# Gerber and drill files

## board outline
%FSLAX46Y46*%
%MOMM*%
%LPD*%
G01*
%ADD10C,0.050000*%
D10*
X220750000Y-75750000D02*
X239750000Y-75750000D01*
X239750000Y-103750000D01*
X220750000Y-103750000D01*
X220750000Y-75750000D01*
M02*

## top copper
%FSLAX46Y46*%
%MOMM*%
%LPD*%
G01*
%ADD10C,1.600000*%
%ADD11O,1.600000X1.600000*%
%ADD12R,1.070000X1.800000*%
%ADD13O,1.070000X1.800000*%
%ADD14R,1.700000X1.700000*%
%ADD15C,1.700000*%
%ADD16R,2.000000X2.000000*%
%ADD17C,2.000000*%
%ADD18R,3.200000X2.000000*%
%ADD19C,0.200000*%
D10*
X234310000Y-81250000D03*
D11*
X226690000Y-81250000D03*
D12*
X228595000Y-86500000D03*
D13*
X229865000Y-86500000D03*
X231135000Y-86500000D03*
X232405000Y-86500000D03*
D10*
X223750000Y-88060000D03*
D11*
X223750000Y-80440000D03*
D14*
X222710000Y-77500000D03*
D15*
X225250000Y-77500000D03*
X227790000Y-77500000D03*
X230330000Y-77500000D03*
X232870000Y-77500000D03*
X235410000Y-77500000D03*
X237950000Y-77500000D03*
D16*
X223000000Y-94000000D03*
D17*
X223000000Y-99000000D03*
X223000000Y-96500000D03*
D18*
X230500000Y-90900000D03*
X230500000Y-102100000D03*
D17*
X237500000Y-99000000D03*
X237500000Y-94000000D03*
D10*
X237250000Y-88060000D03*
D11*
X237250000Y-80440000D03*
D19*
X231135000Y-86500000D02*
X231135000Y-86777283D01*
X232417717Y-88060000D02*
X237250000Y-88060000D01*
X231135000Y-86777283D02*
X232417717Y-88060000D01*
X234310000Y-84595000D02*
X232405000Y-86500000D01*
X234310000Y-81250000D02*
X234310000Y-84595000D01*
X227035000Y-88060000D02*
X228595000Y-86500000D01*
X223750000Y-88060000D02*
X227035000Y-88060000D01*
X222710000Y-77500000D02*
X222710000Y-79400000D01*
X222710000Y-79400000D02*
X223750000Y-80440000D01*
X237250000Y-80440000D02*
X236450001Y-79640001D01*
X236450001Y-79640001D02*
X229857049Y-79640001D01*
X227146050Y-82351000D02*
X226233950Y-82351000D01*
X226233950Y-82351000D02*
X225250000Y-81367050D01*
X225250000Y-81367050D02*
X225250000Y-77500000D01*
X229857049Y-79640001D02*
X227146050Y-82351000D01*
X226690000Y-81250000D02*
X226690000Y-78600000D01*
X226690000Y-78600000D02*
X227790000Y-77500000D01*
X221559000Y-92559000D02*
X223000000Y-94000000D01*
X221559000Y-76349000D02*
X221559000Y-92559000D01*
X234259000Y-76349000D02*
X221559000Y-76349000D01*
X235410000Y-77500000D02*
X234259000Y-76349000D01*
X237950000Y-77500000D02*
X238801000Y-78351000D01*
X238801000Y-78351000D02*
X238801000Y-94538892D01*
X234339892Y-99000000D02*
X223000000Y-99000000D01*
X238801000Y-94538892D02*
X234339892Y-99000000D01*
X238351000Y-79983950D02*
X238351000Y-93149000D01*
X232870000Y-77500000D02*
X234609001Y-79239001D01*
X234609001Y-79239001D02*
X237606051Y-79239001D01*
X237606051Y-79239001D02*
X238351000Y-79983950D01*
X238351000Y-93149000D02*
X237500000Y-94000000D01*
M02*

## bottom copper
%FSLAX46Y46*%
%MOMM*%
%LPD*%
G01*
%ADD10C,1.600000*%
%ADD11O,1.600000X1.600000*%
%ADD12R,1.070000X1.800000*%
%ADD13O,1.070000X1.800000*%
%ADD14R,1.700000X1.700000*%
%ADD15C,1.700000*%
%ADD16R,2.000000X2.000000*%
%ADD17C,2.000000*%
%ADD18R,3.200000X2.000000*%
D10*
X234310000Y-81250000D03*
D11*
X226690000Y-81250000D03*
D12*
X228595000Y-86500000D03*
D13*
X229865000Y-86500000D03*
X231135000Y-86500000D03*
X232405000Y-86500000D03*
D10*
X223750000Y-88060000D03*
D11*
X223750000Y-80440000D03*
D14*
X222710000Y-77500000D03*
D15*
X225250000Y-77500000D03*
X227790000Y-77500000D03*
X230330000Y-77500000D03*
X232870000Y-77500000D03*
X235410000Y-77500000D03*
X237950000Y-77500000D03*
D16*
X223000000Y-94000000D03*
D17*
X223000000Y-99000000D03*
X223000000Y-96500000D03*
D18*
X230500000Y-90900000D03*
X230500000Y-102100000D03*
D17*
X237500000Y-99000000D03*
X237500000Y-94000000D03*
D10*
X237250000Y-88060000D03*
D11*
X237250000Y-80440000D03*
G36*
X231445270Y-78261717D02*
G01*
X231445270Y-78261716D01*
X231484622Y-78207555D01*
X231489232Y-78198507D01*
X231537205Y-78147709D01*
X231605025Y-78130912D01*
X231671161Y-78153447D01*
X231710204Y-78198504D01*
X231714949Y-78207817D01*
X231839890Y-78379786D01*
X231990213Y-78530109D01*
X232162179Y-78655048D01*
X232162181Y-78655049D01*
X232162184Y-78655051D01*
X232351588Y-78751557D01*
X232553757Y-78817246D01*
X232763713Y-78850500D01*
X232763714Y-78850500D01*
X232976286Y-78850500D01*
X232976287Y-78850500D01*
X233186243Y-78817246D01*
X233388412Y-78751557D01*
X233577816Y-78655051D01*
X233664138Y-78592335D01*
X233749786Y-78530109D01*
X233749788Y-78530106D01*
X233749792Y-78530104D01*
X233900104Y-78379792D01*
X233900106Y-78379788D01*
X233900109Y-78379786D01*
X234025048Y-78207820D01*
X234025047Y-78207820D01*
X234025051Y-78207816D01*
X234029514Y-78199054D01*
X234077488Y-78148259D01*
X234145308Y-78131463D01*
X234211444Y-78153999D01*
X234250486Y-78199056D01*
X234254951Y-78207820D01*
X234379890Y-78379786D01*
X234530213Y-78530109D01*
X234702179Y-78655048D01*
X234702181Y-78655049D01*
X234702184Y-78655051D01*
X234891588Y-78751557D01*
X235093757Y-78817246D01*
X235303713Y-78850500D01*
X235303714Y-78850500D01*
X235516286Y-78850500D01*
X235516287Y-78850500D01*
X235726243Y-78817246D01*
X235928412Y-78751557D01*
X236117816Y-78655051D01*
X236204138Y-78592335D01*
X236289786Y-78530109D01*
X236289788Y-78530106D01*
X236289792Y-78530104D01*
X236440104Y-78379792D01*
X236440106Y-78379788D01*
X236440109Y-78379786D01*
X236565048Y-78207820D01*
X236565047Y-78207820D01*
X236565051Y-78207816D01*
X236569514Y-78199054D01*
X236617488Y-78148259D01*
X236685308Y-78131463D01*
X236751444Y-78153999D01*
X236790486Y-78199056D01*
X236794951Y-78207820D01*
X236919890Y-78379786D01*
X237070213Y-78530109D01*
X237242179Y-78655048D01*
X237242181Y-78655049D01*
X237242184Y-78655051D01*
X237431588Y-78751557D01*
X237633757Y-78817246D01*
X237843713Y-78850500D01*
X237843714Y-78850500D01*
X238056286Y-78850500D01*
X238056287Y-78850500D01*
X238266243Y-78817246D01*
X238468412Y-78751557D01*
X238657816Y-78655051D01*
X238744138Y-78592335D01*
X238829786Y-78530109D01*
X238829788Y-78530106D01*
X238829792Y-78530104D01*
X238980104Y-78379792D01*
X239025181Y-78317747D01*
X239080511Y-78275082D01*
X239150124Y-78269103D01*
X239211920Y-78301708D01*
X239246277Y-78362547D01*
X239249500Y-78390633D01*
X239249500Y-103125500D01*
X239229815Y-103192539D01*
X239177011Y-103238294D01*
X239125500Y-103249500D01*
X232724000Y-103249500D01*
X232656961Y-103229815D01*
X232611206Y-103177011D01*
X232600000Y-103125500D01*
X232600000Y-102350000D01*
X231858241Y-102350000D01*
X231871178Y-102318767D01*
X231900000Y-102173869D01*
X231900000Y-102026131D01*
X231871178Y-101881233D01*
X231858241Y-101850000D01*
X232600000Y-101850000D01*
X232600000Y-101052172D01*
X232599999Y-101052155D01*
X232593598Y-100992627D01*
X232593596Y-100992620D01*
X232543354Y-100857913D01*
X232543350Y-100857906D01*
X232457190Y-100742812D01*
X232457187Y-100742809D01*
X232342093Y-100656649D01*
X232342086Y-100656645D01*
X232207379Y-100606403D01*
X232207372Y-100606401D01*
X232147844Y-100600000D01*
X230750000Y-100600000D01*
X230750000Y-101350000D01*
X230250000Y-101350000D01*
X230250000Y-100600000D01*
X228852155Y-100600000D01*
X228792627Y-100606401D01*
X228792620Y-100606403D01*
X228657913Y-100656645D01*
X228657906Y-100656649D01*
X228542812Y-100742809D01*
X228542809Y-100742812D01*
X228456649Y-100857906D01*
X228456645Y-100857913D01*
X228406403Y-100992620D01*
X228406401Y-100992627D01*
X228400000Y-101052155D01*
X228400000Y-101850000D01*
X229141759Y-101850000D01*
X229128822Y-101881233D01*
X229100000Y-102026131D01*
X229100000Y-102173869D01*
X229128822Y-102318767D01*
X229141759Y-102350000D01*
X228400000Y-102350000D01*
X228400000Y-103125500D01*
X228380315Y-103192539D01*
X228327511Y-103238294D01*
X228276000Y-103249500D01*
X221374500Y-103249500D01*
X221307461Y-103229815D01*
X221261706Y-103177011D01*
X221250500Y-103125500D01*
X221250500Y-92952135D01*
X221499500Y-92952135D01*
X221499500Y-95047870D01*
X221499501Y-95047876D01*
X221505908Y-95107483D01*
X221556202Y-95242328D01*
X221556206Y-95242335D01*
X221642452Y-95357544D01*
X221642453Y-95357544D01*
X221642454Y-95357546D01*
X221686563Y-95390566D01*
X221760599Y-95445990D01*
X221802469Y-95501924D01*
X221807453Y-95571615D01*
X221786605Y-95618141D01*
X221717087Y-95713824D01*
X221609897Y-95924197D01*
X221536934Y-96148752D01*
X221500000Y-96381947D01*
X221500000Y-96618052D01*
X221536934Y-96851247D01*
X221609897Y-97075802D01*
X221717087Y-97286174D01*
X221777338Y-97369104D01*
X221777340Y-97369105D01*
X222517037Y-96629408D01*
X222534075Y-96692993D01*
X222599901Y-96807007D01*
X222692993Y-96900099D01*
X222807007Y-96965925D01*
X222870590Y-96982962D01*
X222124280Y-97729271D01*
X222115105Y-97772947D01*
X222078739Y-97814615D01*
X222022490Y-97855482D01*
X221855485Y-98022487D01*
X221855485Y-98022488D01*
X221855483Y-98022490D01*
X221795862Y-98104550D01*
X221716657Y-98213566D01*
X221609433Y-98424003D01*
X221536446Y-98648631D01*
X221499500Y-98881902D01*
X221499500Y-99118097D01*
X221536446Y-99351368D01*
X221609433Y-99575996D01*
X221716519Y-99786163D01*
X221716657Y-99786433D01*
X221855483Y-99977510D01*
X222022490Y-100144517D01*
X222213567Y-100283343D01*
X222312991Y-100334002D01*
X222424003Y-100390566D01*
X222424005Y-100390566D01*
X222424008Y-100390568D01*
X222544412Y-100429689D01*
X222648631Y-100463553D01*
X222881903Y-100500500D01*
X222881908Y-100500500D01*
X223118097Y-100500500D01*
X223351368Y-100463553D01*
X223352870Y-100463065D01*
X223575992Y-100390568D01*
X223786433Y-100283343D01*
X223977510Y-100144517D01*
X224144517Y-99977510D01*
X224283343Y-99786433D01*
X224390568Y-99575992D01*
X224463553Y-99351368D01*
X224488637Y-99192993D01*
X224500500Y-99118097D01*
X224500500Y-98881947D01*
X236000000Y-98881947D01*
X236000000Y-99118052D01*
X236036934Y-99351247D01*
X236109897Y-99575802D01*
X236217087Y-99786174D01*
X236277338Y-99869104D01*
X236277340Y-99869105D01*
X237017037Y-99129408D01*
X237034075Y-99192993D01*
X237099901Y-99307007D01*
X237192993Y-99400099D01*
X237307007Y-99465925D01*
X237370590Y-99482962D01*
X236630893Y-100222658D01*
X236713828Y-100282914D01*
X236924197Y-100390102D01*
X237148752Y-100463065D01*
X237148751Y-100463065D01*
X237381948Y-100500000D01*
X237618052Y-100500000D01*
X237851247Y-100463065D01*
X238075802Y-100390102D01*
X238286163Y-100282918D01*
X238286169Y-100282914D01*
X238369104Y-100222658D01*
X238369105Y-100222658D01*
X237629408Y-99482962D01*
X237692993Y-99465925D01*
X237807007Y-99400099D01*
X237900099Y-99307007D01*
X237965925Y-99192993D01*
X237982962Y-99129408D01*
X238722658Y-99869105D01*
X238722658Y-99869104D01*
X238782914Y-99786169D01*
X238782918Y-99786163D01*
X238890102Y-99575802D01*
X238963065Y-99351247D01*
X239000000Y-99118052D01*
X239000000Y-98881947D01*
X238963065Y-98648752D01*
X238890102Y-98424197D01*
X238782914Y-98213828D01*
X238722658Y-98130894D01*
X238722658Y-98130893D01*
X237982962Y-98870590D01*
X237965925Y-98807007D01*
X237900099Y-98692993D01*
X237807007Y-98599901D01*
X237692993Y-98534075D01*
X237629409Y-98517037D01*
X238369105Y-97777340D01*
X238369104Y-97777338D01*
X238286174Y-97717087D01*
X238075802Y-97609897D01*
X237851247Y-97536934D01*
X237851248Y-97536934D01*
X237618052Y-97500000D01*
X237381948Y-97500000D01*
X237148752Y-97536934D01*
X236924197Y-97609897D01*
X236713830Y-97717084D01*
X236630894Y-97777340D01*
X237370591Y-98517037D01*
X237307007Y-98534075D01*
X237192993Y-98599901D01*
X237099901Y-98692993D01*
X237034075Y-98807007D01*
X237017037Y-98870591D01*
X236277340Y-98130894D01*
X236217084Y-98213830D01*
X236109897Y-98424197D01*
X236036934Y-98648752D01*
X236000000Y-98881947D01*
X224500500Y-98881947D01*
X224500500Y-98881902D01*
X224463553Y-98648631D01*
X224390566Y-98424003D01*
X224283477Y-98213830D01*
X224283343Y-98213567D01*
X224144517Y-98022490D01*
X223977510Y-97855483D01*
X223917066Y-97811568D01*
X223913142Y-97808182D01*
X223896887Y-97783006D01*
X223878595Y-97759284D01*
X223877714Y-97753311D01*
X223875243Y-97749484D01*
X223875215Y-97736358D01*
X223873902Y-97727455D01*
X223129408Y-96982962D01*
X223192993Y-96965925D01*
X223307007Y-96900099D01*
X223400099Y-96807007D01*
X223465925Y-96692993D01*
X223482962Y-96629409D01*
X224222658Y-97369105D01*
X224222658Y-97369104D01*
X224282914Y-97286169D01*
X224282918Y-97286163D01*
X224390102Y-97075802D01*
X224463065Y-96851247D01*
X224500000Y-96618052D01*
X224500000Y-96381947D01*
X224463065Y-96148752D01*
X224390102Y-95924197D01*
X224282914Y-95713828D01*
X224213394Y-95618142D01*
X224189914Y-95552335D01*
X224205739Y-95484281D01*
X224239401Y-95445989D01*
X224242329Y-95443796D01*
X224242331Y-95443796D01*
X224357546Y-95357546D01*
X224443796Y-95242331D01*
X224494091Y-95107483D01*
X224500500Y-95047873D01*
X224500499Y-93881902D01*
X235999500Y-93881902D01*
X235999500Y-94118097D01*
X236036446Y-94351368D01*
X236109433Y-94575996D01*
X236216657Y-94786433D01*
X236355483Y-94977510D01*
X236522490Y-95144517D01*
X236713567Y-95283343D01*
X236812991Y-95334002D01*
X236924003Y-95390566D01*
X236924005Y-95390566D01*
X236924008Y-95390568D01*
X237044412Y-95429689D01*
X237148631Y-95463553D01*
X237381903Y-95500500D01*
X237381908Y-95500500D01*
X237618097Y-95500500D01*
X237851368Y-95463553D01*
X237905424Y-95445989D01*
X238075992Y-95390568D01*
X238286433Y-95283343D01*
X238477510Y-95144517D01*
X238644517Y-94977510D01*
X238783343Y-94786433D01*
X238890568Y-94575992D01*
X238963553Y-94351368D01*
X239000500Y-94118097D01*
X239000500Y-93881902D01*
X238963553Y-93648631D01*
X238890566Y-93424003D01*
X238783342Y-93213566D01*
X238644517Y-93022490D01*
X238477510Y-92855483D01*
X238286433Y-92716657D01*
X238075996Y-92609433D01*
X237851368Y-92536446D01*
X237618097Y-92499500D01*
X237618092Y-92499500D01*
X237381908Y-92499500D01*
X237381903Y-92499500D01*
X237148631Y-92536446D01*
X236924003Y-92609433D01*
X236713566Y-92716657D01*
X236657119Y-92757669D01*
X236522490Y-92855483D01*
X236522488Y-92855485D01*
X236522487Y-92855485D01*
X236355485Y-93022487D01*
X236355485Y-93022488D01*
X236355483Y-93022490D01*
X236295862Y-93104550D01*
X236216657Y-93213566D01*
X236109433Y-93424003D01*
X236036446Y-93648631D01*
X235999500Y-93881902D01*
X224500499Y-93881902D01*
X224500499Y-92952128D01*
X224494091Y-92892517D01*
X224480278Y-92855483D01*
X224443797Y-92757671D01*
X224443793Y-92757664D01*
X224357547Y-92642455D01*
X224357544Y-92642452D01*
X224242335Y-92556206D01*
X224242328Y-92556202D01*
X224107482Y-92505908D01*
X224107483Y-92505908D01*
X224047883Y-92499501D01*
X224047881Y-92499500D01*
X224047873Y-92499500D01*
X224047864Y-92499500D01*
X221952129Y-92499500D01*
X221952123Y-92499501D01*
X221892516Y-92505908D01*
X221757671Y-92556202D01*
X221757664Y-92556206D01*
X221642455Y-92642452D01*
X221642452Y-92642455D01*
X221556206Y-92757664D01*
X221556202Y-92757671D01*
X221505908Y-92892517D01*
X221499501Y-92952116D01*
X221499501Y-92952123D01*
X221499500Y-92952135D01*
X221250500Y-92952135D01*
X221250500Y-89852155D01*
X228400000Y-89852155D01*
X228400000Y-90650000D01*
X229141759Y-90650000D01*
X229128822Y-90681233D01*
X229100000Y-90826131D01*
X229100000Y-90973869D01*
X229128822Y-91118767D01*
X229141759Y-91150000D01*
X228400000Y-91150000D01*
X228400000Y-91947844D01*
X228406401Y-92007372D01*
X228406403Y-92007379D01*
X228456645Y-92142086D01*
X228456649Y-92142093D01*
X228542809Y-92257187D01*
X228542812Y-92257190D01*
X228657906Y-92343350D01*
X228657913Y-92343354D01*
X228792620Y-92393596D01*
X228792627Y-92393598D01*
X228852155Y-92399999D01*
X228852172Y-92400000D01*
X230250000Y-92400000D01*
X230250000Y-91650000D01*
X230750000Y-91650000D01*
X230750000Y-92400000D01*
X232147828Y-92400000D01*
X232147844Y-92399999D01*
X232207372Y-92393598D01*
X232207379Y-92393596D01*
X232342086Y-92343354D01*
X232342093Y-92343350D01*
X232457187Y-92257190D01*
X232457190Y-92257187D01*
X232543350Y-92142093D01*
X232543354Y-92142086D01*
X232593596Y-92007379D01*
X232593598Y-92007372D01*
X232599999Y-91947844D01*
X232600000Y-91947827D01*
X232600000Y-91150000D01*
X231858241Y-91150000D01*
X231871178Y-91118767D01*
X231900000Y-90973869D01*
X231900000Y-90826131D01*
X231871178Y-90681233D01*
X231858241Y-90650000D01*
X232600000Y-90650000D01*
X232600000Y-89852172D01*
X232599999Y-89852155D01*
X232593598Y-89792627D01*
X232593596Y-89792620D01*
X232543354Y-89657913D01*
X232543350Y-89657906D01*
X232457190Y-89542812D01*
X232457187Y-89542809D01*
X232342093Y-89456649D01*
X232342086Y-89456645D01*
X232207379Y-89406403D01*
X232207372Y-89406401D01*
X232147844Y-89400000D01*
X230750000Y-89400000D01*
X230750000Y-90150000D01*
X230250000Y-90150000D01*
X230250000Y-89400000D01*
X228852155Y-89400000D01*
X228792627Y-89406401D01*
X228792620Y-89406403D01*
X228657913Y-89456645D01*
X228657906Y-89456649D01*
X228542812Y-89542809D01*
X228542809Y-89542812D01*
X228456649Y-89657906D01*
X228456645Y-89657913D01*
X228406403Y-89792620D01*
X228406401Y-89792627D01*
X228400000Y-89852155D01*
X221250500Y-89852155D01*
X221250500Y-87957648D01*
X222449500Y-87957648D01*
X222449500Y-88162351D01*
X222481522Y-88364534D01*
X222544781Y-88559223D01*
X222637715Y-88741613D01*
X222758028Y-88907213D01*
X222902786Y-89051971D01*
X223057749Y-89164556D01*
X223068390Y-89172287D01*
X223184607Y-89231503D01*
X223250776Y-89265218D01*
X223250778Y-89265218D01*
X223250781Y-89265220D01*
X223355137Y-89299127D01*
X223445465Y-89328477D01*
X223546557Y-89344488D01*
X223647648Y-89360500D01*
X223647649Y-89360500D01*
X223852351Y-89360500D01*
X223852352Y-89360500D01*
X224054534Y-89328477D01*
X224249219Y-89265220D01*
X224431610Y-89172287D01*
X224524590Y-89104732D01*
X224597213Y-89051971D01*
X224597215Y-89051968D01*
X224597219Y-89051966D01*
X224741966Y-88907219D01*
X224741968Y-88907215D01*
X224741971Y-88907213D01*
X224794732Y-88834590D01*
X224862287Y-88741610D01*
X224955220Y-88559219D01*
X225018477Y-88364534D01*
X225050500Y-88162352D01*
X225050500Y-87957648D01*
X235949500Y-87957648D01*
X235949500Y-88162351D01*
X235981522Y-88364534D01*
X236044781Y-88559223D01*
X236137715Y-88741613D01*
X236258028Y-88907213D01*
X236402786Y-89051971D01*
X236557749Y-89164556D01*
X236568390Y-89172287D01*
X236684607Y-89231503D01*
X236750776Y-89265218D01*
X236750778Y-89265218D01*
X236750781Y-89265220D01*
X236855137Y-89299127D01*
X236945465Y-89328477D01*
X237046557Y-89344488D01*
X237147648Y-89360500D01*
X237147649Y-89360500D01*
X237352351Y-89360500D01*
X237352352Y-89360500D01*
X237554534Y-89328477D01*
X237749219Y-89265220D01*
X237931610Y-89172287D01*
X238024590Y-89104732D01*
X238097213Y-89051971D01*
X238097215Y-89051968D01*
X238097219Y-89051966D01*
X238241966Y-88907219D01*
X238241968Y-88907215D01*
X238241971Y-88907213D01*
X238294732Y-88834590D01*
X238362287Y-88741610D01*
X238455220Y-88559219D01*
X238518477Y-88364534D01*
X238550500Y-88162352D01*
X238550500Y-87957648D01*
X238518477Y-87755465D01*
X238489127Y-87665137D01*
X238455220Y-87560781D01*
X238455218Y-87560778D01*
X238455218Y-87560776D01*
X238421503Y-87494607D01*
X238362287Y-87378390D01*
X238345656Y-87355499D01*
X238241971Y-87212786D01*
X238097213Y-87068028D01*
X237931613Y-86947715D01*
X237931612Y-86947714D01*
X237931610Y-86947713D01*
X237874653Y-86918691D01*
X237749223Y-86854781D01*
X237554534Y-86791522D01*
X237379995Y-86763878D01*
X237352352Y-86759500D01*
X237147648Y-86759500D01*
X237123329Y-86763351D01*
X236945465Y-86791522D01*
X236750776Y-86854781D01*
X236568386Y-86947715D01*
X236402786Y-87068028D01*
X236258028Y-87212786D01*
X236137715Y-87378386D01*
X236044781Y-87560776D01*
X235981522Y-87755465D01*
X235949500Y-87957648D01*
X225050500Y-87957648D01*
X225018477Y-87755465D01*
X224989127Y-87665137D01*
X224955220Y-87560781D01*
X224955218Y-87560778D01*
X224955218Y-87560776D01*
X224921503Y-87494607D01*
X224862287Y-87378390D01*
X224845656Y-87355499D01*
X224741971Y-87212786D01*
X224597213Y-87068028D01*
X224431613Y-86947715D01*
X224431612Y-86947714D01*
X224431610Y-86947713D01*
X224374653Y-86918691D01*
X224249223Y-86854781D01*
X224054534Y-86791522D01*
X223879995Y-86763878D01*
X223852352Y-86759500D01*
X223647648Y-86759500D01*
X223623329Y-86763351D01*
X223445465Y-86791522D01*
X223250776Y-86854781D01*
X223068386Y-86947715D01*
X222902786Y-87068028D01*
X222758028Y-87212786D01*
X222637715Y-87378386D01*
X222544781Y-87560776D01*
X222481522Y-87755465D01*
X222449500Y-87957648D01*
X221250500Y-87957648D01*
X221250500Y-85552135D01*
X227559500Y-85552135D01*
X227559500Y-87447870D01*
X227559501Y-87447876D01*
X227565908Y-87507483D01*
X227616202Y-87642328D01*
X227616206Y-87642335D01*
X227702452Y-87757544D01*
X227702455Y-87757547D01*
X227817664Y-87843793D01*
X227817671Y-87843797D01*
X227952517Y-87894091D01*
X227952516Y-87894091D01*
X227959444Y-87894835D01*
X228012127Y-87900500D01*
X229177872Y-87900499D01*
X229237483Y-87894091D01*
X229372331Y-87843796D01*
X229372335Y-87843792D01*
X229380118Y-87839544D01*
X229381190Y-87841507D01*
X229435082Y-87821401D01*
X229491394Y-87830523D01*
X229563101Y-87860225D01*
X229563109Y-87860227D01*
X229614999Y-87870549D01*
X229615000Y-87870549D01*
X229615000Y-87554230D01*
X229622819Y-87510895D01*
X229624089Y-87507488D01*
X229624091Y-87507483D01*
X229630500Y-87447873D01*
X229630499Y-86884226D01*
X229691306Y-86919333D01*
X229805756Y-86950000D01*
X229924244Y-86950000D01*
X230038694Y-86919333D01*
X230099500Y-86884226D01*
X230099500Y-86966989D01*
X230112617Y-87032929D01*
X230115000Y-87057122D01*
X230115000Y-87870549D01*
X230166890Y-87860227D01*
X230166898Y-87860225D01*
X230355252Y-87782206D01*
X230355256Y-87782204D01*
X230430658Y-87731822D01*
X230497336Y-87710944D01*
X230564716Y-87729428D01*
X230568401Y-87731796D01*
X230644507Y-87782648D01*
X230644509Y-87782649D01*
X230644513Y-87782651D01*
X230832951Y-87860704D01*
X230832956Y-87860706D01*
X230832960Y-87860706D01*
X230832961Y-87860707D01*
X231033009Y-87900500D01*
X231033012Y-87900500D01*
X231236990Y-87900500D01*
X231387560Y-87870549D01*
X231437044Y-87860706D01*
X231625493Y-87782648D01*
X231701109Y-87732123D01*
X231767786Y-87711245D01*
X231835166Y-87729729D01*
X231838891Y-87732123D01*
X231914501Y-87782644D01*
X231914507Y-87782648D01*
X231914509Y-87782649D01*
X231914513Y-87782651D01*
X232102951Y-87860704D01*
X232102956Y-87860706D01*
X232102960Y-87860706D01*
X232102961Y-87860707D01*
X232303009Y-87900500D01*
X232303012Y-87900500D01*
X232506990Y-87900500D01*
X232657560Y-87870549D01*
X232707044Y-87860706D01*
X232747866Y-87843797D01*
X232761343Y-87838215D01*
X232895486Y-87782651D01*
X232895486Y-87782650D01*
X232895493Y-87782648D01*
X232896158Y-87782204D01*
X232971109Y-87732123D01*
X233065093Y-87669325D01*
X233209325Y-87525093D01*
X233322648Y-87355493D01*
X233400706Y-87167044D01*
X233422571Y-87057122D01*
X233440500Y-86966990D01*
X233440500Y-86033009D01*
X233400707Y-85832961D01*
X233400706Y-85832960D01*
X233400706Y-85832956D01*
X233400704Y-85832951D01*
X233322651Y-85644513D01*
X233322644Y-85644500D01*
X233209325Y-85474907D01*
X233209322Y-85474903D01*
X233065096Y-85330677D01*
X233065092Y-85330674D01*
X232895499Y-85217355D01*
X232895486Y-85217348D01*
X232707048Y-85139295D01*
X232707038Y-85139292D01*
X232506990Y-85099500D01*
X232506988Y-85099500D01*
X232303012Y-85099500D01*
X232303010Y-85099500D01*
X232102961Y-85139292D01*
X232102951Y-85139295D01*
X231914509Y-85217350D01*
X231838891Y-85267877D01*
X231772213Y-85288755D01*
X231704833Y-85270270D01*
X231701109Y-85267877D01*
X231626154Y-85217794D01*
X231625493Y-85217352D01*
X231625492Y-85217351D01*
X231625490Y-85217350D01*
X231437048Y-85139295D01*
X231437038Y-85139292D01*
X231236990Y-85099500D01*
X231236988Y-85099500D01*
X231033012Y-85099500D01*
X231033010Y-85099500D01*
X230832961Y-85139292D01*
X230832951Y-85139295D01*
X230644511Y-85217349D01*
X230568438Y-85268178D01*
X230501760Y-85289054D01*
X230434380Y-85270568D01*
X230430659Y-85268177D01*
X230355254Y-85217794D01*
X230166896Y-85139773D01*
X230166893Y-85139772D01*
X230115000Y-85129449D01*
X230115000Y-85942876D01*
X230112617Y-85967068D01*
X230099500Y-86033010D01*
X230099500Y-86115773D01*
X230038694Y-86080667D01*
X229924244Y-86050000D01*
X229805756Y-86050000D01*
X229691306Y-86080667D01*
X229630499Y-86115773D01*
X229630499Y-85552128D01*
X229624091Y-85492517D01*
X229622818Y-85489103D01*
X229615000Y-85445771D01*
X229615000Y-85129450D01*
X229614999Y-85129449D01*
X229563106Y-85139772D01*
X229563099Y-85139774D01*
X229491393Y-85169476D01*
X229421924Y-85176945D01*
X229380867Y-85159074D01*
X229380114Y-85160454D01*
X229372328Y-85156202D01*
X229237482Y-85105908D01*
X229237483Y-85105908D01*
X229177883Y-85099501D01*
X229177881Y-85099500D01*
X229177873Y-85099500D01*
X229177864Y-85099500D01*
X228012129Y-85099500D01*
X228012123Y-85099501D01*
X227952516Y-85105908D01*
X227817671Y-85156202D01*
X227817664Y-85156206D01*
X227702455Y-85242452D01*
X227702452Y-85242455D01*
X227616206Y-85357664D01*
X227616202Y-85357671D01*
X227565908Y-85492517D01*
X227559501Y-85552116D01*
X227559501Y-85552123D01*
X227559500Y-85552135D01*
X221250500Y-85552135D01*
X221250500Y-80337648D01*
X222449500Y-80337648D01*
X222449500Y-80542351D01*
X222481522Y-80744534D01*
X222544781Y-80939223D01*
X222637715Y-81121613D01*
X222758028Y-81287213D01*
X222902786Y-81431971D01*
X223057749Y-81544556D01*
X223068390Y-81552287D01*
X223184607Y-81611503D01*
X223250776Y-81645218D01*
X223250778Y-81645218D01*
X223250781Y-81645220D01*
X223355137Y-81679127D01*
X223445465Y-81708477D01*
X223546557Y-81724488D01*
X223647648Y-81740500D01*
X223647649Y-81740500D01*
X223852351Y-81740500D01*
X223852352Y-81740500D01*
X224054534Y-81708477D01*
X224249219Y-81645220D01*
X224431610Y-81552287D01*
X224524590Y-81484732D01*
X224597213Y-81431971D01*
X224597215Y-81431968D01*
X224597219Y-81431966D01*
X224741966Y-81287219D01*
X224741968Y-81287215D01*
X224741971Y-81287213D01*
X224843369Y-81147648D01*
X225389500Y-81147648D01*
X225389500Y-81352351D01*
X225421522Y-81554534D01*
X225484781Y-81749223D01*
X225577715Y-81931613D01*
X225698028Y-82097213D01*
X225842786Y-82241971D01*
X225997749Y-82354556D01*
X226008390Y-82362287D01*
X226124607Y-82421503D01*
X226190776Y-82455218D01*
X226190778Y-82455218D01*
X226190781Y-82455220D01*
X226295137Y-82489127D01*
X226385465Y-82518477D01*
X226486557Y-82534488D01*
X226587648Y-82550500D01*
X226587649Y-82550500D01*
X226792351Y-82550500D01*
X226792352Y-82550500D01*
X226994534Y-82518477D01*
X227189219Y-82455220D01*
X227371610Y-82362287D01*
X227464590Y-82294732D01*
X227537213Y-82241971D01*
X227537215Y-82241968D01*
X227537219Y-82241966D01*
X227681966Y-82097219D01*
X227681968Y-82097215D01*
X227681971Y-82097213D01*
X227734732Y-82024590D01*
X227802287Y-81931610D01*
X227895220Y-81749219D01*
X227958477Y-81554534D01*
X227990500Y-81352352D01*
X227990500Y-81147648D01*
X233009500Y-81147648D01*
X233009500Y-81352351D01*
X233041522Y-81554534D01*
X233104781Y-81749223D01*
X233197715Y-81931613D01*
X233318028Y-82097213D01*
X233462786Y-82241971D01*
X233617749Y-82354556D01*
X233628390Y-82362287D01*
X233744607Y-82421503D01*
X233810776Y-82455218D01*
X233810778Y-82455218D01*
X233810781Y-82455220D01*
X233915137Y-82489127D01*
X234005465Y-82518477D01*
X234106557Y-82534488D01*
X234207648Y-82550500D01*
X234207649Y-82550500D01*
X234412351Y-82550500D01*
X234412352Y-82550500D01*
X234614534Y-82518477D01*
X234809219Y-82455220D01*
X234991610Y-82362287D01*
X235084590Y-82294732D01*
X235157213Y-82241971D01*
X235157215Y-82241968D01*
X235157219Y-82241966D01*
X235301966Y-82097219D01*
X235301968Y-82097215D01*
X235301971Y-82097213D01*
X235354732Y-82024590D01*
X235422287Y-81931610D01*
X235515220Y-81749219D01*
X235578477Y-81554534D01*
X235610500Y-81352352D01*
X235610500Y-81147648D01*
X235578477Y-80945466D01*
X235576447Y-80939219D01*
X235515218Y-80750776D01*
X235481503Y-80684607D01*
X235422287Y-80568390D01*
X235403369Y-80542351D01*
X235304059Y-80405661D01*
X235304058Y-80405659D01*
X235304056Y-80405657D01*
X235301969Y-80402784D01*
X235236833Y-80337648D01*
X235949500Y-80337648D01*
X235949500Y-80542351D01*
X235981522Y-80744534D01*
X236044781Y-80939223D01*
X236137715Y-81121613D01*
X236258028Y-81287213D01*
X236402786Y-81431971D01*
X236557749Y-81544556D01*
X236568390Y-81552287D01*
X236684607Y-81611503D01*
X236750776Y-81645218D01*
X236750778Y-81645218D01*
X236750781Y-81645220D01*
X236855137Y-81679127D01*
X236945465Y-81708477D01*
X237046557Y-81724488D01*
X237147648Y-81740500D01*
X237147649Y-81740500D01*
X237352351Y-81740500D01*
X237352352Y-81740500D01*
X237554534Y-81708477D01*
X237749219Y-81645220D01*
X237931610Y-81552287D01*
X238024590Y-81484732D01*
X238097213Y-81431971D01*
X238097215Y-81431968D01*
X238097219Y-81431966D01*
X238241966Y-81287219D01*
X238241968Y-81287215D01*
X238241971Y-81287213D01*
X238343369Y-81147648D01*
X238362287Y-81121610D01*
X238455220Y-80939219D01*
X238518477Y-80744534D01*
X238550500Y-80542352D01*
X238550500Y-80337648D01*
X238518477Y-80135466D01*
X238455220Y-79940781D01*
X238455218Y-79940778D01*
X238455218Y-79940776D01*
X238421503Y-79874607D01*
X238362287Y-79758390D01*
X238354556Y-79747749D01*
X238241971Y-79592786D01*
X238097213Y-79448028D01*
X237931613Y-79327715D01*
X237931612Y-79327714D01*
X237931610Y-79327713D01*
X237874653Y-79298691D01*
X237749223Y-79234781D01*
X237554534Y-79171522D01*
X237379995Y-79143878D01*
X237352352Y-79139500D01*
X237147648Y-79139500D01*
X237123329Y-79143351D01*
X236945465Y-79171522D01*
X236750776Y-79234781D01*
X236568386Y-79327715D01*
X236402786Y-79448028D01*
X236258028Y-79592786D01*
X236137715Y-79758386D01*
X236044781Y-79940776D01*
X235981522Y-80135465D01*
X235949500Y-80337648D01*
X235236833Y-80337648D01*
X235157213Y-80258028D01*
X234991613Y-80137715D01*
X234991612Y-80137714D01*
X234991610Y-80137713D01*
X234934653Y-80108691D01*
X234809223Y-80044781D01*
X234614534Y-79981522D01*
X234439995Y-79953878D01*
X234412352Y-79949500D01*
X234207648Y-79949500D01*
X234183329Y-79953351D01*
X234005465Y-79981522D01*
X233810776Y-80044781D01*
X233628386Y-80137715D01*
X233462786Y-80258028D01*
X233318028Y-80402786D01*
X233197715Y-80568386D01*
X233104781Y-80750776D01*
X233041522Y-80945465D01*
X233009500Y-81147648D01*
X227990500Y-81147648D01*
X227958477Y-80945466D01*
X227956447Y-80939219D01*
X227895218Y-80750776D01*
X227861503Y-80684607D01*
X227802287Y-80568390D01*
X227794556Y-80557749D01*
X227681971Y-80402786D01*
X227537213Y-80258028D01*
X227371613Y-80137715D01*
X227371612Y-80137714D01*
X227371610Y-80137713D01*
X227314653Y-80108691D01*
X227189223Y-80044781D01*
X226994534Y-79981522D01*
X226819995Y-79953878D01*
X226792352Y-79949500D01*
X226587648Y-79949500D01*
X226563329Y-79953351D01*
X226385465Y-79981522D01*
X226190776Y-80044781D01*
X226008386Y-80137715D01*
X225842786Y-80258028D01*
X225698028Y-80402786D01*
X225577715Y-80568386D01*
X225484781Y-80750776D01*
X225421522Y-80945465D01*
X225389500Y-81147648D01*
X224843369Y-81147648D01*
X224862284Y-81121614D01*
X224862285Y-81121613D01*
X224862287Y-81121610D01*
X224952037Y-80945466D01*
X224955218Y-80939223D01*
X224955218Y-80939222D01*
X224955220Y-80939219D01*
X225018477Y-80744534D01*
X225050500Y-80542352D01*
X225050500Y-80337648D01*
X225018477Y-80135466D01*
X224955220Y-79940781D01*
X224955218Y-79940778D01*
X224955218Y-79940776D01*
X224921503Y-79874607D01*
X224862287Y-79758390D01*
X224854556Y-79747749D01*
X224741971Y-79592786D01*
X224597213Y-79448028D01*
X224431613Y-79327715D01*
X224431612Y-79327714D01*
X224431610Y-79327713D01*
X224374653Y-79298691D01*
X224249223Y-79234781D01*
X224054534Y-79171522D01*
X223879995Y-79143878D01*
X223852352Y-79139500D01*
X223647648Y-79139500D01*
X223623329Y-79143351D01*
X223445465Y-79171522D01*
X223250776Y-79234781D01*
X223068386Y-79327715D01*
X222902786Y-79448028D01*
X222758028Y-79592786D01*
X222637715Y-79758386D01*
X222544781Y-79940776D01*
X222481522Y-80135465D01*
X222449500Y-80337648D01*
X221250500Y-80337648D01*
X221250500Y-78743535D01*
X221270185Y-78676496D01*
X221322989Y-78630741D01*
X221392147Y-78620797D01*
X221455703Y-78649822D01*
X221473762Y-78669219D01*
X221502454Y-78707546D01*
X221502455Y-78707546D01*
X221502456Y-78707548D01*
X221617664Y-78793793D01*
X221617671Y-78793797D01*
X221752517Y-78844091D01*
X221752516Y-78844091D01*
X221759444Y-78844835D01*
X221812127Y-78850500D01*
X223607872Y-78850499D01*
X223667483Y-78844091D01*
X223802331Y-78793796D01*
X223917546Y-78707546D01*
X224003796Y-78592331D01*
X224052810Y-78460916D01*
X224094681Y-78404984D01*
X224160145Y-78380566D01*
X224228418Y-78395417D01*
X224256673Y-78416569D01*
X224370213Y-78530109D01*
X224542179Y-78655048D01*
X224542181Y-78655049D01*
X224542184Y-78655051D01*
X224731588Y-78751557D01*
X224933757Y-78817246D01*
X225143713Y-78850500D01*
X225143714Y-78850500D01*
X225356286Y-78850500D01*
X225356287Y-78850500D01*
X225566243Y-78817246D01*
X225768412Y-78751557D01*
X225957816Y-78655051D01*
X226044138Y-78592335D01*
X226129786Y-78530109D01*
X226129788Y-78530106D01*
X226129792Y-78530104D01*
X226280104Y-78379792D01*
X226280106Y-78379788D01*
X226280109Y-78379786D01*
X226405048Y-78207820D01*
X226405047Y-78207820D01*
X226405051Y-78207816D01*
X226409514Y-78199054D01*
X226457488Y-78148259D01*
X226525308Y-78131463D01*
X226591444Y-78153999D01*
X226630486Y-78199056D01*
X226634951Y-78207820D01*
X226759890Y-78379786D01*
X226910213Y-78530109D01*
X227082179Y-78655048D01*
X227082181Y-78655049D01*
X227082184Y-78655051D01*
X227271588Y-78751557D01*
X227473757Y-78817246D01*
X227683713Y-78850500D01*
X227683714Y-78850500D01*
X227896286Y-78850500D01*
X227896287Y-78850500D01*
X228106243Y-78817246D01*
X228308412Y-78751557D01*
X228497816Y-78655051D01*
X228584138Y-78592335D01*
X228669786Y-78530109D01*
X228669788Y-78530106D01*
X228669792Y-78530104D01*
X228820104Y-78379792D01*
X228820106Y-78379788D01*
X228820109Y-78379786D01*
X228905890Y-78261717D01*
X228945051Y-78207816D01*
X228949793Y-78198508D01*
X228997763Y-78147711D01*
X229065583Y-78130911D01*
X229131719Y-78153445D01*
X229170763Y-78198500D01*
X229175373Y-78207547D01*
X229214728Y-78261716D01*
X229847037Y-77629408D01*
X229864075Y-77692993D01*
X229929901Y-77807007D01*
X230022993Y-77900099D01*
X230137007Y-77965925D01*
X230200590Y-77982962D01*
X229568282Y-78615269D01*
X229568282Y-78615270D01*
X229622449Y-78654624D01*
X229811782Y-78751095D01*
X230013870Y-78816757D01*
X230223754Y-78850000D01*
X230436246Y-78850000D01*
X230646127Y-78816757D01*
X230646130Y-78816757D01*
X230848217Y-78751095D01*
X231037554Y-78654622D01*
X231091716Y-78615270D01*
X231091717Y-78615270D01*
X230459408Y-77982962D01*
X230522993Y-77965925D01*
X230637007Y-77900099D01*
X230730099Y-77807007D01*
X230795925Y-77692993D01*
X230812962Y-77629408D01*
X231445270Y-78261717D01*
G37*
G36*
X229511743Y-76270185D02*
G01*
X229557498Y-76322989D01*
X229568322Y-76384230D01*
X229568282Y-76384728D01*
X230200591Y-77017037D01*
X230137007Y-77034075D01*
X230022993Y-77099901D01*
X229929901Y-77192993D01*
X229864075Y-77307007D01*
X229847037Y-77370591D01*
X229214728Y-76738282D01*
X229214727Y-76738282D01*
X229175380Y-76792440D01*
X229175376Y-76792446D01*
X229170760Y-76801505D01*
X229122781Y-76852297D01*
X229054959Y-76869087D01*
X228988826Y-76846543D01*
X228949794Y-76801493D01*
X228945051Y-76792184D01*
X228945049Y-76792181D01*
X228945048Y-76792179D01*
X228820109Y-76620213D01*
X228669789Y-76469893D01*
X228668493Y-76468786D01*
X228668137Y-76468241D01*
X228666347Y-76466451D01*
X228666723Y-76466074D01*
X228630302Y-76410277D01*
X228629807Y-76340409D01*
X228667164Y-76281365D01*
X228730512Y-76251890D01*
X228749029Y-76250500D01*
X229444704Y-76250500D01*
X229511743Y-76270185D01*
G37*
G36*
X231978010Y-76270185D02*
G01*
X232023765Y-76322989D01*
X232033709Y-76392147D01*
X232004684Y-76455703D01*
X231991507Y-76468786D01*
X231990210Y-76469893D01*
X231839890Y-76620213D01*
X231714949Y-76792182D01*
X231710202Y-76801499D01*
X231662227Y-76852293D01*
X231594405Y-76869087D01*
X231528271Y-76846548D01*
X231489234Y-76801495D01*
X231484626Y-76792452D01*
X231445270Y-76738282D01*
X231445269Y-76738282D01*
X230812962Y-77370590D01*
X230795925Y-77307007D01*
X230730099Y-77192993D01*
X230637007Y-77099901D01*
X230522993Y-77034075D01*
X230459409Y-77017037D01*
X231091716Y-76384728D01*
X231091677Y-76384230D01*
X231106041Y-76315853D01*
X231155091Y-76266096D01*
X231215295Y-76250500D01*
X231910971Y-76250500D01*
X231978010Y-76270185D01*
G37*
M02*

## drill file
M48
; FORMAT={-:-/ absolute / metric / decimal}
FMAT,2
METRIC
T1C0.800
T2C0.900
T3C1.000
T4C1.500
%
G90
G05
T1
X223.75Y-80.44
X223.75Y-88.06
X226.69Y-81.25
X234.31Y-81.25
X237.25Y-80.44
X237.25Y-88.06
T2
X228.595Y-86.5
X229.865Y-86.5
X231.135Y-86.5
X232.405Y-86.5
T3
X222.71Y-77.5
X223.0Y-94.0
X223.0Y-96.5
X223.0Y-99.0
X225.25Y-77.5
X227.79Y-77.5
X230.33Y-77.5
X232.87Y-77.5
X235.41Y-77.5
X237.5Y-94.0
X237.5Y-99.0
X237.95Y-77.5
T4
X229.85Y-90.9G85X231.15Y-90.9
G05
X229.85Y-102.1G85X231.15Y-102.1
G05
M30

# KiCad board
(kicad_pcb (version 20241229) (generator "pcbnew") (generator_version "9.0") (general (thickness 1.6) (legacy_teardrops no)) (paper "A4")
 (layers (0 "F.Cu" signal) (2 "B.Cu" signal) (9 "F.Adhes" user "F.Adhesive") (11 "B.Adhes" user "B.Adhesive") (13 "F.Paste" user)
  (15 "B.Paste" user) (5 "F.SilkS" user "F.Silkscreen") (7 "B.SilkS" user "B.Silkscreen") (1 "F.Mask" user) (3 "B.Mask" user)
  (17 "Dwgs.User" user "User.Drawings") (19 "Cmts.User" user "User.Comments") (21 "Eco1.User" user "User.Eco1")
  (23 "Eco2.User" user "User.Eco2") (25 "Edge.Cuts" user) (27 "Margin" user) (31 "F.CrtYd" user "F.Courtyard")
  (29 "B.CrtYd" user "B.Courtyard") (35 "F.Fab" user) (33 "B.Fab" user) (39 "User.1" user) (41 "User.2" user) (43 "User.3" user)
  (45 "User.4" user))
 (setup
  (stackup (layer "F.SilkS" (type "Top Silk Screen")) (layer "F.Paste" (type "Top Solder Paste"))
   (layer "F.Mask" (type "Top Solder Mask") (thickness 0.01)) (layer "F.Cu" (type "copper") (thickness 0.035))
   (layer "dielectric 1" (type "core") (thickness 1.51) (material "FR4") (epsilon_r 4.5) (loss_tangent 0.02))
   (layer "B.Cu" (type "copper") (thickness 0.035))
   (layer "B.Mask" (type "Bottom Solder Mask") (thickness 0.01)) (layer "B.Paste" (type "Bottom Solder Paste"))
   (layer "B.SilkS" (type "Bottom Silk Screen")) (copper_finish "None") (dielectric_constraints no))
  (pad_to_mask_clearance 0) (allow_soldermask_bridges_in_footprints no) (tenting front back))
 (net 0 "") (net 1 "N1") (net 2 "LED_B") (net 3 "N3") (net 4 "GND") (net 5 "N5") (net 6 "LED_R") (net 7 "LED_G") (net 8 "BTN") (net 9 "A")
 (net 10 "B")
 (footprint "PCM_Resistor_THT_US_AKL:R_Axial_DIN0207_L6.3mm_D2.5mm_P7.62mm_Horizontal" (layer "F.Cu") (at 234.31 81.25 180)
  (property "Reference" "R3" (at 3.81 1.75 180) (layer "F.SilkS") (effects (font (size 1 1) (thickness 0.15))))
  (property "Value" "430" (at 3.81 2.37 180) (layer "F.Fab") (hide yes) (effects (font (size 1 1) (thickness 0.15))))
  (pad "1" thru_hole circle (at 0 0 180) (size 1.6 1.6) (drill 0.8) (layers "*.Cu" "*.Mask") (remove_unused_layers no) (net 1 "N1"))
  (pad "2" thru_hole oval (at 7.62 0 180) (size 1.6 1.6) (drill 0.8) (layers "*.Cu" "*.Mask") (remove_unused_layers no) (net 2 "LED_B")))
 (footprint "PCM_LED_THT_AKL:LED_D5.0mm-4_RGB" (layer "F.Cu") (at 230.5 86.5)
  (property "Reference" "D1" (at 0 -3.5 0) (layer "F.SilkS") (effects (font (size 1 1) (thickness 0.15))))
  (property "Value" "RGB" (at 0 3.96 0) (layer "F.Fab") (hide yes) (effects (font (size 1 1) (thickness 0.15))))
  (pad "1" thru_hole rect (at -1.905 0) (size 1.07 1.8) (drill 0.9) (layers "*.Cu" "*.Mask") (remove_unused_layers no) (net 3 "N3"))
  (pad "2" thru_hole oval (at -0.635 0) (size 1.07 1.8) (drill 0.9) (layers "*.Cu" "*.Mask") (remove_unused_layers no) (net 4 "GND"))
  (pad "3" thru_hole oval (at 0.635 0) (size 1.07 1.8) (drill 0.9) (layers "*.Cu" "*.Mask") (remove_unused_layers no) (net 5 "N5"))
  (pad "4" thru_hole oval (at 1.905 0) (size 1.07 1.8) (drill 0.9) (layers "*.Cu" "*.Mask") (remove_unused_layers no) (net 1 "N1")))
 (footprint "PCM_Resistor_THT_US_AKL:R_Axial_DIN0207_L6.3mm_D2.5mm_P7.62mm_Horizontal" (layer "F.Cu") (at 223.75 88.06 90)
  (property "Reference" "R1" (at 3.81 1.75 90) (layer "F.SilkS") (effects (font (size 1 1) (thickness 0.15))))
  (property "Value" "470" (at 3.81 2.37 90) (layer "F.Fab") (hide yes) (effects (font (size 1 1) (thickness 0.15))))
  (pad "1" thru_hole circle (at 0 0 90) (size 1.6 1.6) (drill 0.8) (layers "*.Cu" "*.Mask") (remove_unused_layers no) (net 3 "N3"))
  (pad "2" thru_hole oval (at 7.62 0 90) (size 1.6 1.6) (drill 0.8) (layers "*.Cu" "*.Mask") (remove_unused_layers no) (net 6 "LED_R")))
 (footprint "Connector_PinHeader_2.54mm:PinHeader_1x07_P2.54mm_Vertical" (layer "F.Cu") (at 222.71 77.5 90)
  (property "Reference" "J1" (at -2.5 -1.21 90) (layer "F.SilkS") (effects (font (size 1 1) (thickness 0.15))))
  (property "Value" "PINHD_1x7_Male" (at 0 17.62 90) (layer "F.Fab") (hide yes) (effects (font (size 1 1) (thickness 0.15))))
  (pad "1" thru_hole rect (at 0 0 90) (size 1.7 1.7) (drill 1) (layers "*.Cu" "*.Mask") (remove_unused_layers no) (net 6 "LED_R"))
  (pad "2" thru_hole circle (at 0 2.54 90) (size 1.7 1.7) (drill 1) (layers "*.Cu" "*.Mask") (remove_unused_layers no) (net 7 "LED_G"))
  (pad "3" thru_hole circle (at 0 5.08 90) (size 1.7 1.7) (drill 1) (layers "*.Cu" "*.Mask") (remove_unused_layers no) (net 2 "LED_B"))
  (pad "4" thru_hole circle (at 0 7.62 90) (size 1.7 1.7) (drill 1) (layers "*.Cu" "*.Mask") (remove_unused_layers no) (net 4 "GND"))
  (pad "5" thru_hole circle (at 0 10.16 90) (size 1.7 1.7) (drill 1) (layers "*.Cu" "*.Mask") (remove_unused_layers no) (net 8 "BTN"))
  (pad "6" thru_hole circle (at 0 12.7 90) (size 1.7 1.7) (drill 1) (layers "*.Cu" "*.Mask") (remove_unused_layers no) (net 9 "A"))
  (pad "7" thru_hole circle (at 0 15.24 90) (size 1.7 1.7) (drill 1) (layers "*.Cu" "*.Mask") (remove_unused_layers no) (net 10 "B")))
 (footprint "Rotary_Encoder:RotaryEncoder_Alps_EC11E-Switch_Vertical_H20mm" (layer "F.Cu") (at 230.5 96.5)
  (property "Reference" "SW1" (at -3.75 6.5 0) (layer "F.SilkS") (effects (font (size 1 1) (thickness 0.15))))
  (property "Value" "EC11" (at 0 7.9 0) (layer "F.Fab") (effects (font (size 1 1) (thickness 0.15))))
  (pad "A" thru_hole rect (at -7.5 -2.5) (size 2 2) (drill 1) (layers "*.Cu" "*.Mask") (remove_unused_layers no) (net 9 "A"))
  (pad "B" thru_hole circle (at -7.5 2.5) (size 2 2) (drill 1) (layers "*.Cu" "*.Mask") (remove_unused_layers no) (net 10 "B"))
  (pad "C" thru_hole circle (at -7.5 0) (size 2 2) (drill 1) (layers "*.Cu" "*.Mask") (remove_unused_layers no) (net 4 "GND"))
  (pad "MP" thru_hole rect (at 0 -5.6) (size 3.2 2) (drill oval 2.8 1.5) (layers "*.Cu" "*.Mask") (remove_unused_layers no) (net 4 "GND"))
  (pad "MP" thru_hole rect (at 0 5.6) (size 3.2 2) (drill oval 2.8 1.5) (layers "*.Cu" "*.Mask") (remove_unused_layers no) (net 4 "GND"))
  (pad "S1" thru_hole circle (at 7 2.5) (size 2 2) (drill 1) (layers "*.Cu" "*.Mask") (remove_unused_layers no) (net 4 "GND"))
  (pad "S2" thru_hole circle (at 7 -2.5) (size 2 2) (drill 1) (layers "*.Cu" "*.Mask") (remove_unused_layers no) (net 8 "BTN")))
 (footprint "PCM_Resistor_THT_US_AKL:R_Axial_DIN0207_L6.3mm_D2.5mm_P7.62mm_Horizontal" (layer "F.Cu") (at 237.25 88.06 90)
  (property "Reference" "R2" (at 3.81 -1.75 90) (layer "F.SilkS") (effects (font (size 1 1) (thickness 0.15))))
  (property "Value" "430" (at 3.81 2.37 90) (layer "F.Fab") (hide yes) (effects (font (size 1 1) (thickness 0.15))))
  (pad "1" thru_hole circle (at 0 0 90) (size 1.6 1.6) (drill 0.8) (layers "*.Cu" "*.Mask") (remove_unused_layers no) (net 5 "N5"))
  (pad "2" thru_hole oval (at 7.62 0 90) (size 1.6 1.6) (drill 0.8) (layers "*.Cu" "*.Mask") (remove_unused_layers no) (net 7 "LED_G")))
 (gr_rect (start 220.75 75.75) (end 239.75 103.75) (stroke (width 0.05) (type default)) (fill no) (layer "Edge.Cuts"))
 (segment (start 231.135 86.5) (end 231.135 86.777283) (width 0.2) (layer "F.Cu") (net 5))
 (segment (start 232.417717 88.06) (end 237.25 88.06) (width 0.2) (layer "F.Cu") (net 5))
 (segment (start 231.135 86.777283) (end 232.417717 88.06) (width 0.2) (layer "F.Cu") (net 5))
 (segment (start 234.31 84.595) (end 232.405 86.5) (width 0.2) (layer "F.Cu") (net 1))
 (segment (start 234.31 81.25) (end 234.31 84.595) (width 0.2) (layer "F.Cu") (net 1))
 (segment (start 227.035 88.06) (end 228.595 86.5) (width 0.2) (layer "F.Cu") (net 3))
 (segment (start 223.75 88.06) (end 227.035 88.06) (width 0.2) (layer "F.Cu") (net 3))
 (segment (start 222.71 77.5) (end 222.71 79.4) (width 0.2) (layer "F.Cu") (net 6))
 (segment (start 222.71 79.4) (end 223.75 80.44) (width 0.2) (layer "F.Cu") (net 6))
 (segment (start 237.25 80.44) (end 236.450001 79.640001) (width 0.2) (layer "F.Cu") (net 7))
 (segment (start 236.450001 79.640001) (end 229.857049 79.640001) (width 0.2) (layer "F.Cu") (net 7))
 (segment (start 227.14605 82.351) (end 226.23395 82.351) (width 0.2) (layer "F.Cu") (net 7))
 (segment (start 226.23395 82.351) (end 225.25 81.36705) (width 0.2) (layer "F.Cu") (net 7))
 (segment (start 225.25 81.36705) (end 225.25 77.5) (width 0.2) (layer "F.Cu") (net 7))
 (segment (start 229.857049 79.640001) (end 227.14605 82.351) (width 0.2) (layer "F.Cu") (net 7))
 (segment (start 226.69 81.25) (end 226.69 78.6) (width 0.2) (layer "F.Cu") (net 2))
 (segment (start 226.69 78.6) (end 227.79 77.5) (width 0.2) (layer "F.Cu") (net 2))
 (segment (start 221.559 92.559) (end 223 94) (width 0.2) (layer "F.Cu") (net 9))
 (segment (start 221.559 76.349) (end 221.559 92.559) (width 0.2) (layer "F.Cu") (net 9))
 (segment (start 234.259 76.349) (end 221.559 76.349) (width 0.2) (layer "F.Cu") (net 9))
 (segment (start 235.41 77.5) (end 234.259 76.349) (width 0.2) (layer "F.Cu") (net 9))
 (segment (start 237.95 77.5) (end 238.801 78.351) (width 0.2) (layer "F.Cu") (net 10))
 (segment (start 238.801 78.351) (end 238.801 94.538892) (width 0.2) (layer "F.Cu") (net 10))
 (segment (start 234.339892 99) (end 223 99) (width 0.2) (layer "F.Cu") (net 10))
 (segment (start 238.801 94.538892) (end 234.339892 99) (width 0.2) (layer "F.Cu") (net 10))
 (segment (start 238.351 79.98395) (end 238.351 93.149) (width 0.2) (layer "F.Cu") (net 8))
 (segment (start 232.87 77.5) (end 234.609001 79.239001) (width 0.2) (layer "F.Cu") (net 8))
 (segment (start 234.609001 79.239001) (end 237.606051 79.239001) (width 0.2) (layer "F.Cu") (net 8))
 (segment (start 237.606051 79.239001) (end 238.351 79.98395) (width 0.2) (layer "F.Cu") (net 8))
 (segment (start 238.351 93.149) (end 237.5 94) (width 0.2) (layer "F.Cu") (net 8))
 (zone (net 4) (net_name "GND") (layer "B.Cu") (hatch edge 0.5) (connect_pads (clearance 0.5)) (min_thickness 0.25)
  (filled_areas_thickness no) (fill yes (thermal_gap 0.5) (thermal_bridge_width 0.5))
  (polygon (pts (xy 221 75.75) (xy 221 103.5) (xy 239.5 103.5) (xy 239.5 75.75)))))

